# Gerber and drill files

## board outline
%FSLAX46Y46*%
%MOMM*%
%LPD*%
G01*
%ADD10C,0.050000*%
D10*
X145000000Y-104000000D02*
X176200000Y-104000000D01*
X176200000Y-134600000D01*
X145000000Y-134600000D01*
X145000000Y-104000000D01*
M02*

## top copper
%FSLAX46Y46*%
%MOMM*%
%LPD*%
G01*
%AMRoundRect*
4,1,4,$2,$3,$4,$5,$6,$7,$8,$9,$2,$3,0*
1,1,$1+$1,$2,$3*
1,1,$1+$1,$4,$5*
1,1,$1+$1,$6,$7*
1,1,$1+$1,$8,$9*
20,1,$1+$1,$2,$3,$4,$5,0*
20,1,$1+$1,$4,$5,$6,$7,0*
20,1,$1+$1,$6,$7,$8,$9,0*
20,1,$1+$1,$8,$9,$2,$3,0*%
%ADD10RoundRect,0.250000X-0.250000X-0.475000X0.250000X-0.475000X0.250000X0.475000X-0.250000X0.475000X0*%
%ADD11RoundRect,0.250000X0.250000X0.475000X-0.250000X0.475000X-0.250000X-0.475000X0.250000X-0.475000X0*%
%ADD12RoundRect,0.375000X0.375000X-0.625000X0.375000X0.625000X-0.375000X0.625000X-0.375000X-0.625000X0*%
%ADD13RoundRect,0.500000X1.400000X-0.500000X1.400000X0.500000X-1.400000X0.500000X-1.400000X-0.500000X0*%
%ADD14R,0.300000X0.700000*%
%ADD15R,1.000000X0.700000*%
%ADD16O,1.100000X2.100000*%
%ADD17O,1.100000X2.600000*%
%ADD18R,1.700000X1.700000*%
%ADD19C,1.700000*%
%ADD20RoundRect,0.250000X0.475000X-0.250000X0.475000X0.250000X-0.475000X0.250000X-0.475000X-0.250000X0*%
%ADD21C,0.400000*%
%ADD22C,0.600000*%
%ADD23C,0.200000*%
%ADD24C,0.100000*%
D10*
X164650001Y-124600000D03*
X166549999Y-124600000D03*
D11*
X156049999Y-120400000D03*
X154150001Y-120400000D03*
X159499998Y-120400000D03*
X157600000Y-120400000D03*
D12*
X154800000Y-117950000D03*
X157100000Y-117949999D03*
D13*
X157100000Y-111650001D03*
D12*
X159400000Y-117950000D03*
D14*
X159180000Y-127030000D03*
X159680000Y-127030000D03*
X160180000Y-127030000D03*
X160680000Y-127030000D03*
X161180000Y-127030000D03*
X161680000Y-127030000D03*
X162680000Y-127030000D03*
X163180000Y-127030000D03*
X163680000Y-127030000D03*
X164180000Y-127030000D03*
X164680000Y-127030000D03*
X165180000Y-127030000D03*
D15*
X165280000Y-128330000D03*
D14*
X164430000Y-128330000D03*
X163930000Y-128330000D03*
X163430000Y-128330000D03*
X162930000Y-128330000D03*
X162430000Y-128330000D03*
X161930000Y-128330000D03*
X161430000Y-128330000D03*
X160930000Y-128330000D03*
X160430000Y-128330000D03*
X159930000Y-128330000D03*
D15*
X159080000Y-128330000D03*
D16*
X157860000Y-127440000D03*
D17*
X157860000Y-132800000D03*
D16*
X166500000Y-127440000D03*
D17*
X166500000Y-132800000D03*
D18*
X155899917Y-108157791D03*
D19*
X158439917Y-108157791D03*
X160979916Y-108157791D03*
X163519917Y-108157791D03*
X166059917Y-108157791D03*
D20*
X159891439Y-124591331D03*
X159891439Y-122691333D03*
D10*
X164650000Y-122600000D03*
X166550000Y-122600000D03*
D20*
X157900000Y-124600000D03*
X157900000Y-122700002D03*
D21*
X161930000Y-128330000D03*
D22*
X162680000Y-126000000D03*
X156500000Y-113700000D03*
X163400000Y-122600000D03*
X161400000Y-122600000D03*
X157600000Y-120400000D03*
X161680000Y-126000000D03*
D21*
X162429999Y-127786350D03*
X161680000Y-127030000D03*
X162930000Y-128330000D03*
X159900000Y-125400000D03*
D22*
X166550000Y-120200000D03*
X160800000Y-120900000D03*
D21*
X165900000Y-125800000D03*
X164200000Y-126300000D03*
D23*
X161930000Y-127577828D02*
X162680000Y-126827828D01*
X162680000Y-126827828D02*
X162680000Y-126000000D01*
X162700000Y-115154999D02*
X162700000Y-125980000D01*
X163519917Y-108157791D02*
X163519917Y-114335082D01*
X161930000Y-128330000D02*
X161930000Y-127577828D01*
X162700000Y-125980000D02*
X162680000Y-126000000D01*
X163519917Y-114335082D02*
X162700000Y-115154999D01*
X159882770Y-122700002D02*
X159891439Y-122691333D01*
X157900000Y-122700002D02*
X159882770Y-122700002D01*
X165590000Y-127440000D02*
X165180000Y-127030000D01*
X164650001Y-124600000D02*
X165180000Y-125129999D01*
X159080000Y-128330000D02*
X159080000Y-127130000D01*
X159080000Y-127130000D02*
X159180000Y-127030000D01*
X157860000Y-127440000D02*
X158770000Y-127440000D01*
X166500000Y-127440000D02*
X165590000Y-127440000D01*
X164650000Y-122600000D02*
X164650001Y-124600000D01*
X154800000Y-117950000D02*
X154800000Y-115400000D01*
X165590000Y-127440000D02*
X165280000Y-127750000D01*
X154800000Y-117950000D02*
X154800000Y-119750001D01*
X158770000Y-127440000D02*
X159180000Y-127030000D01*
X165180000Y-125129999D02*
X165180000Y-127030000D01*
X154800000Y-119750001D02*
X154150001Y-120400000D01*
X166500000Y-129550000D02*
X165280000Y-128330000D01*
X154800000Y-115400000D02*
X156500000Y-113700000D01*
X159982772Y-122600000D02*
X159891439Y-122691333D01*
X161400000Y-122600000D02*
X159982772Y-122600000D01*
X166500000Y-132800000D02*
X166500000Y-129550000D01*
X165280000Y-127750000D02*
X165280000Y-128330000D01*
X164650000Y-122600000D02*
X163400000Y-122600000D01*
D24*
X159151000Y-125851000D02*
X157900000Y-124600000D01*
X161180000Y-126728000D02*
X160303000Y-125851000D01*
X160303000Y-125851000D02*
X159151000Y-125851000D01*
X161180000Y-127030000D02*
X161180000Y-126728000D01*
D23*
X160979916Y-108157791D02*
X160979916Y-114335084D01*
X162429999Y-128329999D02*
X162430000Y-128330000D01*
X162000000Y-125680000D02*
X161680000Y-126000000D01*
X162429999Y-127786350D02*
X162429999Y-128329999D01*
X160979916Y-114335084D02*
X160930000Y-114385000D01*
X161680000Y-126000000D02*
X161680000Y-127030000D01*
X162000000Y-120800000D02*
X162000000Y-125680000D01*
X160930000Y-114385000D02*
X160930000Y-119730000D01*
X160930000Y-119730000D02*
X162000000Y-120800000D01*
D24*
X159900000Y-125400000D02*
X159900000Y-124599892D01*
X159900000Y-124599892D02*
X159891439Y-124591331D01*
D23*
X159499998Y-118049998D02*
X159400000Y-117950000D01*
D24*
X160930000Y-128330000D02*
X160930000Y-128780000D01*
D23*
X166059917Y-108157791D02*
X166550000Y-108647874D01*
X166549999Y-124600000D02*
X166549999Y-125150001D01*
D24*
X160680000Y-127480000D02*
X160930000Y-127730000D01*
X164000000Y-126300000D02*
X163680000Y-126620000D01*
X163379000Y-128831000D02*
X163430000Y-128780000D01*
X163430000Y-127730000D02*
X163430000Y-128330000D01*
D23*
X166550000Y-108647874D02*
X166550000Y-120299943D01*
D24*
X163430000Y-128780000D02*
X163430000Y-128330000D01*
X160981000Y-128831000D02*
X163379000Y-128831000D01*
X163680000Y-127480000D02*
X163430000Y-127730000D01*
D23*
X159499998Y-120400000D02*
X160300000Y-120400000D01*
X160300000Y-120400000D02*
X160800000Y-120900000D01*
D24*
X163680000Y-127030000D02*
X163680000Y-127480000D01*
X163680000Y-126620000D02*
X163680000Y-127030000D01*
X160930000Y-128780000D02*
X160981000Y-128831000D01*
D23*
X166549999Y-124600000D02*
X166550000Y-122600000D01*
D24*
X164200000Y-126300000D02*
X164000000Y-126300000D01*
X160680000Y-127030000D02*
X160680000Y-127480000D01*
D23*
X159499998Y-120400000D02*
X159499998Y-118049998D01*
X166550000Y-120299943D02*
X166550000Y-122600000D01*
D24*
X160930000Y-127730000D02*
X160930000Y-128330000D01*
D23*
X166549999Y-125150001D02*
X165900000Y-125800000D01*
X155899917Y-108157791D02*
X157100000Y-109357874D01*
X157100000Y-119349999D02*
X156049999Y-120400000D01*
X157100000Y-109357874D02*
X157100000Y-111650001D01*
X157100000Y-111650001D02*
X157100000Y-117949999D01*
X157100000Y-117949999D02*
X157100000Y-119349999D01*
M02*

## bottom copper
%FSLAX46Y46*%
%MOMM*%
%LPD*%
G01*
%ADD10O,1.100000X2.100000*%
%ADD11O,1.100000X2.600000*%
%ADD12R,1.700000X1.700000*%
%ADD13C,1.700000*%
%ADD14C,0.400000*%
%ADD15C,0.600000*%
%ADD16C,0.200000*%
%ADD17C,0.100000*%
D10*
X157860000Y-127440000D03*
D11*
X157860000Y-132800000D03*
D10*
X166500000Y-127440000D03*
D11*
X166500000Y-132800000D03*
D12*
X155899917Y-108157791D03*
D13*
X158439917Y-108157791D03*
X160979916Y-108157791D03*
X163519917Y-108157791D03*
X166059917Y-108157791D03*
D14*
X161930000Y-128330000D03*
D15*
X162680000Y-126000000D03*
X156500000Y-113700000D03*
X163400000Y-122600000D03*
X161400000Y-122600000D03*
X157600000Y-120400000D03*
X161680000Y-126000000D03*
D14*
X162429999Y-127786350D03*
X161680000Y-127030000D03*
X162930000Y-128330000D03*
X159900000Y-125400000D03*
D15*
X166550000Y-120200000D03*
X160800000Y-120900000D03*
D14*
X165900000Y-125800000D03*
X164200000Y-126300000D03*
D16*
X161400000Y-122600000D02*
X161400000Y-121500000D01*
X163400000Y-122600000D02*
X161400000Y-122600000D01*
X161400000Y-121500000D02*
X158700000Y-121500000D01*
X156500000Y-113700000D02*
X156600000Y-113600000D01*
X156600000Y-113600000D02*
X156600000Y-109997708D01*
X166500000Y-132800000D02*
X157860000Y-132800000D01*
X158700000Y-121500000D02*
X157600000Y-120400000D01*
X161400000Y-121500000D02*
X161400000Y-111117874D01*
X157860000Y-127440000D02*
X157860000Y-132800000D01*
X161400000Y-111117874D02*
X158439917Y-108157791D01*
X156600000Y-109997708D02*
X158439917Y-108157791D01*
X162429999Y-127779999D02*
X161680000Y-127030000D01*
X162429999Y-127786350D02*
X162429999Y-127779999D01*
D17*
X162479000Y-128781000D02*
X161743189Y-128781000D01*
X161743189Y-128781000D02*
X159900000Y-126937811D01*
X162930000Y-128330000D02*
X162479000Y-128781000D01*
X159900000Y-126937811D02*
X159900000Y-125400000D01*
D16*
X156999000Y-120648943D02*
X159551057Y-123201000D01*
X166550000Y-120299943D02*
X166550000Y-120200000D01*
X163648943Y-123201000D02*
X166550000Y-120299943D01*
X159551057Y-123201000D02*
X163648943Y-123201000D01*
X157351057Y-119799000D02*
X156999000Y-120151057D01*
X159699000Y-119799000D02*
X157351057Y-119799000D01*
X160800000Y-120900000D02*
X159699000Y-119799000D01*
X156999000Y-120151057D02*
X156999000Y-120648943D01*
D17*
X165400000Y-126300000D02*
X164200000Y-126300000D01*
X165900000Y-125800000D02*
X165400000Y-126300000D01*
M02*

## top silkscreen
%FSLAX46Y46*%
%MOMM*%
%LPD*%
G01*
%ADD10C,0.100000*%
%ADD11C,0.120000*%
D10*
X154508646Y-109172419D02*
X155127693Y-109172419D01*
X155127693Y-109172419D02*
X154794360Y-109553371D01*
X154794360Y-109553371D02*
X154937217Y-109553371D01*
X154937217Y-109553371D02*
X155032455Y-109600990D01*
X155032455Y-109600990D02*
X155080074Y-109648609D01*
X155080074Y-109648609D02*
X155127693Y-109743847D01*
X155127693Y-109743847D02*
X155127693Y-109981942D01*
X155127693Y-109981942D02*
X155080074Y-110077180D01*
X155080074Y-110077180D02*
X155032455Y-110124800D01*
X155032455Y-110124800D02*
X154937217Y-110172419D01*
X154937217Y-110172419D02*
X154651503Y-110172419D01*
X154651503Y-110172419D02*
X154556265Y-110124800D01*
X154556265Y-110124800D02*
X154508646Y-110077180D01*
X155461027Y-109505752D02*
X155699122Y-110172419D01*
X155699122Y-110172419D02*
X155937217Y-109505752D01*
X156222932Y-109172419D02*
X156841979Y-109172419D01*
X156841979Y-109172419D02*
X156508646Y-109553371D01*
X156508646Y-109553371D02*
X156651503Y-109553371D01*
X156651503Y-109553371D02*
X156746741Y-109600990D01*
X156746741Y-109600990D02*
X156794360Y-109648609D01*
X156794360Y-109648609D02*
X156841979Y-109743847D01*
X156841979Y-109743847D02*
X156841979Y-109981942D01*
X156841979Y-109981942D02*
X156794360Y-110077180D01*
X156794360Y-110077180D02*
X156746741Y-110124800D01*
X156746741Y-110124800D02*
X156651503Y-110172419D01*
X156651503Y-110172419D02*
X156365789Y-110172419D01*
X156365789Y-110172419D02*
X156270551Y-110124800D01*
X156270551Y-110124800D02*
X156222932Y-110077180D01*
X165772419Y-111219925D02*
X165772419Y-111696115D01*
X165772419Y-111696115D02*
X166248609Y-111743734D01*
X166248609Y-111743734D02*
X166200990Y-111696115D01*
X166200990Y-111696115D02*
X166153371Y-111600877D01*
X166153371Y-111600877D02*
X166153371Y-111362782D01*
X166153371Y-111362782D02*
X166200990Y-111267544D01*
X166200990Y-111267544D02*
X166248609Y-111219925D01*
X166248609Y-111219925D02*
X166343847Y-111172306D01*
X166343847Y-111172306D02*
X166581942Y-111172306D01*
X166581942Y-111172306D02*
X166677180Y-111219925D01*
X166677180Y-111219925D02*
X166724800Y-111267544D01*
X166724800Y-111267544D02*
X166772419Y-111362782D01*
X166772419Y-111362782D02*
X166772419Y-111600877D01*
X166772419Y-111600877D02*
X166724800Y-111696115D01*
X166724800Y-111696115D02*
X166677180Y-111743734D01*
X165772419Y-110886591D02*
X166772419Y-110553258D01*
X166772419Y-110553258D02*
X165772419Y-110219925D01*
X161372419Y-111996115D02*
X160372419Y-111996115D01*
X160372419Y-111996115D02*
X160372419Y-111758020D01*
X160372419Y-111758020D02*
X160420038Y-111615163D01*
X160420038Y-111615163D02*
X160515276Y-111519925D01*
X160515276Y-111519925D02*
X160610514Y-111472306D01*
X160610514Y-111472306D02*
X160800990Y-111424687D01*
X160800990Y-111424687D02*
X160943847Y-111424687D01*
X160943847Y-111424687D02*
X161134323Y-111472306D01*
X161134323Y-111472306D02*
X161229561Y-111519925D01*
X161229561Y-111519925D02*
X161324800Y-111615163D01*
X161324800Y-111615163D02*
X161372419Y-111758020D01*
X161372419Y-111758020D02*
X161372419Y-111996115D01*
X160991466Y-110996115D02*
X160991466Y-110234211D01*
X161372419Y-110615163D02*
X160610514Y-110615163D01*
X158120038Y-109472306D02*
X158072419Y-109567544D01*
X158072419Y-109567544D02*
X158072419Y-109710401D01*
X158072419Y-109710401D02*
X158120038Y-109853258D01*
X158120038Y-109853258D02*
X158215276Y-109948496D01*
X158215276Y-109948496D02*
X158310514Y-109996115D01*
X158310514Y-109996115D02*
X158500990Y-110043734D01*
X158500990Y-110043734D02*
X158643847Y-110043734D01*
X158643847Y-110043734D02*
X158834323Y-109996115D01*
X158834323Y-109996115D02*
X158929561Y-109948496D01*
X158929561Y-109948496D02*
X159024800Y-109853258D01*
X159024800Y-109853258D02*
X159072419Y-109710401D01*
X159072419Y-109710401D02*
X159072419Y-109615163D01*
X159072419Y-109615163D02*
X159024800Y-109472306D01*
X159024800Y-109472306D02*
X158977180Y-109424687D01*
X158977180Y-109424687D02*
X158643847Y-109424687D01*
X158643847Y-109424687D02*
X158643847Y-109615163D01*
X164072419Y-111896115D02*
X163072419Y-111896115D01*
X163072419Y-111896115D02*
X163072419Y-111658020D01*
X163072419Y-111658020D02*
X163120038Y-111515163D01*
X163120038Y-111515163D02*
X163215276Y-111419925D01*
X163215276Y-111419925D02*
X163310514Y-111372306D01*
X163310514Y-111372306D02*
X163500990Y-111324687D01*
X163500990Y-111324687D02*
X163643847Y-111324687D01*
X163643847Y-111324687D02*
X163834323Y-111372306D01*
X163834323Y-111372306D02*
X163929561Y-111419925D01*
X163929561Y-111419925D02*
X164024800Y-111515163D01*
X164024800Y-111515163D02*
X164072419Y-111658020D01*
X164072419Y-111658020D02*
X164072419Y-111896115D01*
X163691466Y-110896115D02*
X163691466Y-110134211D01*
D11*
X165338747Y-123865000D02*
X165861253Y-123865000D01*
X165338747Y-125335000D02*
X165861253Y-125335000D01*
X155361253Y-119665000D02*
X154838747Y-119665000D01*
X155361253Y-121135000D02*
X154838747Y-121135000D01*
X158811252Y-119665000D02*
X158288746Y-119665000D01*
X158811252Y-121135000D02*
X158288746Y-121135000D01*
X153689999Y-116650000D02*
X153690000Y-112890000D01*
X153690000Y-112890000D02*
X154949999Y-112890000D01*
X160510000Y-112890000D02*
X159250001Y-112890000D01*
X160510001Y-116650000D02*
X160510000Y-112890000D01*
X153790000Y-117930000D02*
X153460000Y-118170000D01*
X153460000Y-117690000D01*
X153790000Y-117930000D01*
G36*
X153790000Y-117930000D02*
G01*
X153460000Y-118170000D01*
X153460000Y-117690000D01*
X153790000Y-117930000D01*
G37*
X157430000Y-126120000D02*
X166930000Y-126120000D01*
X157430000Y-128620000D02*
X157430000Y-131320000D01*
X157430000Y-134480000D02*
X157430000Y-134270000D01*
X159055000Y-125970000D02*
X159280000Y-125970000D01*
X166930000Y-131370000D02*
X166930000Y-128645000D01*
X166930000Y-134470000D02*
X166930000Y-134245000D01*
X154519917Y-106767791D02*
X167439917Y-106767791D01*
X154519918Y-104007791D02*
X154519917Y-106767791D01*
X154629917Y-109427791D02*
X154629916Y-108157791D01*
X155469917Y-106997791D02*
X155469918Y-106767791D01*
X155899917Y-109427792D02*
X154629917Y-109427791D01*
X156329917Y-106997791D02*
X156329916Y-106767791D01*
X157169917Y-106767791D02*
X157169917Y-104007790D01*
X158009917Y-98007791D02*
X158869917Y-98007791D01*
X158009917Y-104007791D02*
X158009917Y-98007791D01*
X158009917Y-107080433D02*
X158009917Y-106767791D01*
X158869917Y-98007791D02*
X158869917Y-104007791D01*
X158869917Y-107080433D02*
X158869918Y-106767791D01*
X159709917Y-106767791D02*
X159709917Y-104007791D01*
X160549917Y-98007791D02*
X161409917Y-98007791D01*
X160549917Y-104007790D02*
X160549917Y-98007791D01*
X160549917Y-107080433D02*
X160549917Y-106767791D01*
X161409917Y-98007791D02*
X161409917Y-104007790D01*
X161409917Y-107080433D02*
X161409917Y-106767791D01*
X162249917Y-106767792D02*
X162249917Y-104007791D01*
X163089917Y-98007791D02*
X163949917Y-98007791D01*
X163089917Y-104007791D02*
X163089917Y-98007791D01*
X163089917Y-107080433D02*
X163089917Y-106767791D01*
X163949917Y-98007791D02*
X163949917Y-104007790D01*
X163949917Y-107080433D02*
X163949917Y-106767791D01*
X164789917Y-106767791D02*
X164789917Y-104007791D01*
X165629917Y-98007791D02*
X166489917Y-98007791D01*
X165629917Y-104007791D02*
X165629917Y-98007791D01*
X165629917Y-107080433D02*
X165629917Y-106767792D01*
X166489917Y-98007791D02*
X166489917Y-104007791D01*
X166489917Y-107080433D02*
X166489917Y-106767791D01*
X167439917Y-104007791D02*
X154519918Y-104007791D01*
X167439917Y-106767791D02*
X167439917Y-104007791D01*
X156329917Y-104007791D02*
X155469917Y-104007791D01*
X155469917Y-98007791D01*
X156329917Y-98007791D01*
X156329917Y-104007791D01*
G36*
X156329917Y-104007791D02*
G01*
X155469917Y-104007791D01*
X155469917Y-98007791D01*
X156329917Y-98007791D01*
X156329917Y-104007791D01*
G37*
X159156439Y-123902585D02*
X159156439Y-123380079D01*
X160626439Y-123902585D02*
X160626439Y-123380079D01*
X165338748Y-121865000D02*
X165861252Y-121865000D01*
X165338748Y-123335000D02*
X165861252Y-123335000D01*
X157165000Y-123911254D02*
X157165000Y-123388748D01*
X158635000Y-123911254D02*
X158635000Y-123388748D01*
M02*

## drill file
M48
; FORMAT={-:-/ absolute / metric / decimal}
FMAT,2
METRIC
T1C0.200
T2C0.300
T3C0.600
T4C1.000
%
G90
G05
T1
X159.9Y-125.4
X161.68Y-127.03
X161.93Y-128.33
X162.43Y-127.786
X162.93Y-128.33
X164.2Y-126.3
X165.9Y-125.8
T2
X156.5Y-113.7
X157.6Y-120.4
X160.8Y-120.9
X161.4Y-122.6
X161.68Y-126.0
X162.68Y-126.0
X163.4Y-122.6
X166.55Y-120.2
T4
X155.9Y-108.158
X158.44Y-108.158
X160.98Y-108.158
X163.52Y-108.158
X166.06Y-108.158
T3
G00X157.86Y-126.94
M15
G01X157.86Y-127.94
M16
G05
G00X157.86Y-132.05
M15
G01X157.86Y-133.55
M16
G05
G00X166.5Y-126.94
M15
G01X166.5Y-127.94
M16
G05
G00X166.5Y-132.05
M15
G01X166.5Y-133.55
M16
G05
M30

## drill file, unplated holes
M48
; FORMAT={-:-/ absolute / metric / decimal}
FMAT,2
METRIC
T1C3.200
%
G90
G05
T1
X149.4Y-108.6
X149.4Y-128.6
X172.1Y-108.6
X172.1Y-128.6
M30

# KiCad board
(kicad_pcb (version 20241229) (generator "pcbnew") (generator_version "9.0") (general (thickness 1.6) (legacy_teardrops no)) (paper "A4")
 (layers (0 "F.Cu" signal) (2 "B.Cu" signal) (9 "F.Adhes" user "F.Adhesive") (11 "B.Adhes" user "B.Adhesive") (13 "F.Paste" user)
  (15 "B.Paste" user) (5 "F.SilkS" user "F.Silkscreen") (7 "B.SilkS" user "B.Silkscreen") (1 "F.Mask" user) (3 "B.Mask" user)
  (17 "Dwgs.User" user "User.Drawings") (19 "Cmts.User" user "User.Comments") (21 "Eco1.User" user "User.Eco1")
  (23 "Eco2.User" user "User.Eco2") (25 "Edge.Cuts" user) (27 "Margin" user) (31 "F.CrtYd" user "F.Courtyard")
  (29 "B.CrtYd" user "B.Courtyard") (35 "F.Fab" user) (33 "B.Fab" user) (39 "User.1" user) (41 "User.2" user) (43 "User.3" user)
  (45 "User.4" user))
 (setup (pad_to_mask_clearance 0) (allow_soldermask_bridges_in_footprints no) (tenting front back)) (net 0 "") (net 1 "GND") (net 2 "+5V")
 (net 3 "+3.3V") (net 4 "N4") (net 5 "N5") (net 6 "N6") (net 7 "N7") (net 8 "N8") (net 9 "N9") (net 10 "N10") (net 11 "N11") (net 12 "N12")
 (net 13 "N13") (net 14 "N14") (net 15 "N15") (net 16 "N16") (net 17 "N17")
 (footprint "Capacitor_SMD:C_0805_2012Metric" (layer "F.Cu") (at 165.6 124.6)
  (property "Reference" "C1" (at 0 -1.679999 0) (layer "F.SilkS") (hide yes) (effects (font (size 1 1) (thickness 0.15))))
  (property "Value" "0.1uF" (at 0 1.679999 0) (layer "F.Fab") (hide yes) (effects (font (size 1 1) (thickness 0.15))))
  (fp_line (start -0.261253 -0.735) (end 0.261253 -0.735) (stroke (width 0.12) (type solid)) (layer "F.SilkS"))
  (fp_line (start -0.261253 0.735) (end 0.261253 0.735) (stroke (width 0.12) (type solid)) (layer "F.SilkS"))
  (pad "1" smd roundrect (at -0.949999 0) (size 1 1.45) (layers "F.Cu" "F.Mask" "F.Paste") (roundrect_rratio 0.25) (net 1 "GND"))
  (pad "2" smd roundrect (at 0.949999 0) (size 1 1.45) (layers "F.Cu" "F.Mask" "F.Paste") (roundrect_rratio 0.25) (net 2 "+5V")))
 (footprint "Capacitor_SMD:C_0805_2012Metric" (layer "F.Cu") (at 155.1 120.4 180)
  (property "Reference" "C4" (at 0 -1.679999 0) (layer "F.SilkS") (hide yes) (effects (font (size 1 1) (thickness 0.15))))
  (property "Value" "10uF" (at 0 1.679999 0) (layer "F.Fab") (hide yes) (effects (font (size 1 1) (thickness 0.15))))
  (fp_line (start -0.261253 0.735) (end 0.261253 0.735) (stroke (width 0.12) (type solid)) (layer "F.SilkS"))
  (fp_line (start -0.261253 -0.735) (end 0.261253 -0.735) (stroke (width 0.12) (type solid)) (layer "F.SilkS"))
  (pad "1" smd roundrect (at -0.949999 0 180) (size 1 1.45) (layers "F.Cu" "F.Mask" "F.Paste") (roundrect_rratio 0.25) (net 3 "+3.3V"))
  (pad "2" smd roundrect (at 0.949999 0 180) (size 1 1.45) (layers "F.Cu" "F.Mask" "F.Paste") (roundrect_rratio 0.25) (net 1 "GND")))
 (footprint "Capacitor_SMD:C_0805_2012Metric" (layer "F.Cu") (at 158.549999 120.4 180)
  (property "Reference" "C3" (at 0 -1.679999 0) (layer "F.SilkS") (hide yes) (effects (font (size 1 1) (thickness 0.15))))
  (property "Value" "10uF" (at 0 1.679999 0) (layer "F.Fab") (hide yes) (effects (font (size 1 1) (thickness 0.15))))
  (fp_line (start -0.261253 0.735) (end 0.261253 0.735) (stroke (width 0.12) (type solid)) (layer "F.SilkS"))
  (fp_line (start -0.261253 -0.735) (end 0.261253 -0.735) (stroke (width 0.12) (type solid)) (layer "F.SilkS"))
  (pad "1" smd roundrect (at -0.949999 0 180) (size 1 1.45) (layers "F.Cu" "F.Mask" "F.Paste") (roundrect_rratio 0.25) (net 2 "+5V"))
  (pad "2" smd roundrect (at 0.949999 0 180) (size 1 1.45) (layers "F.Cu" "F.Mask" "F.Paste") (roundrect_rratio 0.25) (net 1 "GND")))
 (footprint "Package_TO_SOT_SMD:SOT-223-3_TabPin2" (layer "F.Cu") (at 157.1 114.8 90)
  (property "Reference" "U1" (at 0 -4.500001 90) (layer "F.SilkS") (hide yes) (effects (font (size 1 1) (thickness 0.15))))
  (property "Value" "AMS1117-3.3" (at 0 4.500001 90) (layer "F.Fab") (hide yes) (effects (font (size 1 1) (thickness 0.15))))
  (fp_line (start -1.85 -3.410001) (end 1.91 -3.41) (stroke (width 0.12) (type solid)) (layer "F.SilkS"))
  (fp_line (start 1.91 -3.41) (end 1.91 -2.150001) (stroke (width 0.12) (type solid)) (layer "F.SilkS"))
  (fp_line (start 1.91 3.41) (end 1.91 2.150001) (stroke (width 0.12) (type solid)) (layer "F.SilkS"))
  (fp_line (start -1.85 3.410001) (end 1.91 3.41) (stroke (width 0.12) (type solid)) (layer "F.SilkS"))
  (fp_poly
   (pts (xy -3.13 -3.31) (xy -3.37 -3.64) (xy -2.89 -3.64) (xy -3.13 -3.31)) (stroke (width 0.12) (type solid)) (fill yes) (layer "F.SilkS"))
  (pad "1" smd roundrect (at -3.15 -2.3 90) (size 2 1.5) (layers "F.Cu" "F.Mask" "F.Paste") (roundrect_rratio 0.25) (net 1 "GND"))
  (pad "2" smd roundrect (at -3.149999 0 90) (size 2 1.5) (layers "F.Cu" "F.Mask" "F.Paste") (roundrect_rratio 0.25) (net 3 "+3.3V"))
  (pad "2" smd roundrect (at 3.149999 0 90) (size 2 3.8) (layers "F.Cu" "F.Mask" "F.Paste") (roundrect_rratio 0.25) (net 3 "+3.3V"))
  (pad "3" smd roundrect (at -3.15 2.3 90) (size 2 1.5) (layers "F.Cu" "F.Mask" "F.Paste") (roundrect_rratio 0.25) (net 2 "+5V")))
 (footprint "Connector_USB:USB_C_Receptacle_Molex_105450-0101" (layer "F.Cu") (at 162.18 130.245)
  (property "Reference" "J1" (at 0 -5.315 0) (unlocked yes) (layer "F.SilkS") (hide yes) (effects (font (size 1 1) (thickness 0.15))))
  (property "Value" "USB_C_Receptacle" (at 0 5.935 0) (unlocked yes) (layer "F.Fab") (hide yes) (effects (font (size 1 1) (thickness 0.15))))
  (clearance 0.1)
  (fp_line (start -4.75 -4.125) (end 4.75 -4.125) (stroke (width 0.12) (type solid)) (layer "F.SilkS"))
  (fp_line (start -4.75 -1.625) (end -4.75 1.075) (stroke (width 0.12) (type solid)) (layer "F.SilkS"))
  (fp_line (start -4.75 4.235) (end -4.75 4.025) (stroke (width 0.12) (type solid)) (layer "F.SilkS"))
  (fp_line (start -3.125 -4.275) (end -2.9 -4.275) (stroke (width 0.12) (type solid)) (layer "F.SilkS"))
  (fp_line (start 4.75 1.125) (end 4.75 -1.6) (stroke (width 0.12) (type solid)) (layer "F.SilkS"))
  (fp_line (start 4.75 4.225) (end 4.75 4) (stroke (width 0.12) (type solid)) (layer "F.SilkS"))
  (pad "A1" smd rect (at -3 -3.215) (size 0.3 0.7) (layers "F.Cu" "F.Mask" "F.Paste") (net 1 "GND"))
  (pad "A2" smd rect (at -2.5 -3.215) (size 0.3 0.7) (layers "F.Cu" "F.Mask" "F.Paste") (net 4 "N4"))
  (pad "A3" smd rect (at -2 -3.215) (size 0.3 0.7) (layers "F.Cu" "F.Mask" "F.Paste") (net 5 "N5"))
  (pad "A4" smd rect (at -1.5 -3.215) (size 0.3 0.7) (layers "F.Cu" "F.Mask" "F.Paste") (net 2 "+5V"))
  (pad "A5" smd rect (at -1 -3.215) (size 0.3 0.7) (layers "F.Cu" "F.Mask" "F.Paste") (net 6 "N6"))
  (pad "A6" smd rect (at -0.5 -3.215) (size 0.3 0.7) (layers "F.Cu" "F.Mask" "F.Paste") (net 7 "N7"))
  (pad "A7" smd rect (at 0.5 -3.215) (size 0.3 0.7) (layers "F.Cu" "F.Mask" "F.Paste") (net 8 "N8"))
  (pad "A8" smd rect (at 1 -3.215) (size 0.3 0.7) (layers "F.Cu" "F.Mask" "F.Paste") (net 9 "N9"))
  (pad "A9" smd rect (at 1.5 -3.215) (size 0.3 0.7) (layers "F.Cu" "F.Mask" "F.Paste") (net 2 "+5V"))
  (pad "A10" smd rect (at 2 -3.215) (size 0.3 0.7) (layers "F.Cu" "F.Mask" "F.Paste") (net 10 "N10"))
  (pad "A11" smd rect (at 2.5 -3.215) (size 0.3 0.7) (layers "F.Cu" "F.Mask" "F.Paste") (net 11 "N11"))
  (pad "A12" smd rect (at 3 -3.215) (size 0.3 0.7) (layers "F.Cu" "F.Mask" "F.Paste") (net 1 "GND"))
  (pad "B1" smd rect (at 3.1 -1.915) (size 1 0.7) (layers "F.Cu" "F.Mask" "F.Paste") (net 1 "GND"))
  (pad "B2" smd rect (at 2.25 -1.915) (size 0.3 0.7) (layers "F.Cu" "F.Mask" "F.Paste") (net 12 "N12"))
  (pad "B3" smd rect (at 1.75 -1.915) (size 0.3 0.7) (layers "F.Cu" "F.Mask" "F.Paste") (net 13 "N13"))
  (pad "B4" smd rect (at 1.25 -1.915) (size 0.3 0.7) (layers "F.Cu" "F.Mask" "F.Paste") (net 2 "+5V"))
  (pad "B5" smd rect (at 0.75 -1.915) (size 0.3 0.7) (layers "F.Cu" "F.Mask" "F.Paste") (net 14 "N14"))
  (pad "B6" smd rect (at 0.25 -1.915) (size 0.3 0.7) (layers "F.Cu" "F.Mask" "F.Paste") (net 7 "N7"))
  (pad "B7" smd rect (at -0.25 -1.915) (size 0.3 0.7) (layers "F.Cu" "F.Mask" "F.Paste") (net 8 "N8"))
  (pad "B8" smd rect (at -0.75 -1.915) (size 0.3 0.7) (layers "F.Cu" "F.Mask" "F.Paste") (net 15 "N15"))
  (pad "B9" smd rect (at -1.25 -1.915) (size 0.3 0.7) (layers "F.Cu" "F.Mask" "F.Paste") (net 2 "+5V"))
  (pad "B10" smd rect (at -1.75 -1.915) (size 0.3 0.7) (layers "F.Cu" "F.Mask" "F.Paste") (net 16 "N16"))
  (pad "B11" smd rect (at -2.25 -1.915) (size 0.3 0.7) (layers "F.Cu" "F.Mask" "F.Paste") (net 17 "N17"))
  (pad "B12" smd rect (at -3.1 -1.915) (size 1 0.7) (layers "F.Cu" "F.Mask" "F.Paste") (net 1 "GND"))
  (pad "S1" thru_hole oval (at -4.32 -2.805) (size 1.1 2.1) (drill oval 0.6 1.6) (layers "*.Cu" "*.Mask") (remove_unused_layers no)
   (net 1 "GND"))
  (pad "S1" thru_hole oval (at -4.32 2.555) (size 1.1 2.6) (drill oval 0.6 2.1) (layers "*.Cu" "*.Mask") (remove_unused_layers no)
   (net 1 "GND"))
  (pad "S1" thru_hole oval (at 4.32 -2.805) (size 1.1 2.1) (drill oval 0.6 1.6) (layers "*.Cu" "*.Mask") (remove_unused_layers no)
   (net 1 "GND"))
  (pad "S1" thru_hole oval (at 4.32 2.555) (size 1.1 2.6) (drill oval 0.6 2.1) (layers "*.Cu" "*.Mask") (remove_unused_layers no)
   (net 1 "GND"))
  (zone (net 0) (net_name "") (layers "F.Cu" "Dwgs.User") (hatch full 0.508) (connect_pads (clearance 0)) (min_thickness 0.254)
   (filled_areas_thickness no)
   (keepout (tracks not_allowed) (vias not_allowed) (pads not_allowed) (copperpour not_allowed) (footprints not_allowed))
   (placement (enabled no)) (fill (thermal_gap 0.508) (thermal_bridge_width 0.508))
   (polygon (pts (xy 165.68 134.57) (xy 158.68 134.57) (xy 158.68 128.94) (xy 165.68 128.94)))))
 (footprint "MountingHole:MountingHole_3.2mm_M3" (layer "F.Cu") (at 172.1 108.6)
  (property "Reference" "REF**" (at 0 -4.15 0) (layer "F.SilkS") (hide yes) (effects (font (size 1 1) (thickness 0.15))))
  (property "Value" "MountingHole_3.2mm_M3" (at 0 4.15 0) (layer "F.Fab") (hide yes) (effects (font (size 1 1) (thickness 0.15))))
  (pad "" np_thru_hole circle (at 0 0) (size 3.2 3.2) (drill 3.2) (layers "*.Cu" "*.Mask")))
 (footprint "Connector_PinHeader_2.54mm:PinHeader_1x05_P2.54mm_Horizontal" (layer "F.Cu") (at 155.899917 108.157791 90)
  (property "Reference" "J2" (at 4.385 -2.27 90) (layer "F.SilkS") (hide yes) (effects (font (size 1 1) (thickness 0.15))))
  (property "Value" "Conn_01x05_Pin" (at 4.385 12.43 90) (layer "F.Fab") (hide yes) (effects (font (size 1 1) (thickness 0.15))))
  (fp_line (start 1.39 -1.38) (end 1.39 11.54) (stroke (width 0.12) (type solid)) (layer "F.SilkS"))
  (fp_line (start 4.15 -1.379999) (end 1.39 -1.38) (stroke (width 0.12) (type solid)) (layer "F.SilkS"))
  (fp_line (start -1.27 -1.27) (end 0 -1.270001) (stroke (width 0.12) (type solid)) (layer "F.SilkS"))
  (fp_line (start 1.16 -0.43) (end 1.39 -0.429999) (stroke (width 0.12) (type solid)) (layer "F.SilkS"))
  (fp_line (start -1.270001 0) (end -1.27 -1.27) (stroke (width 0.12) (type solid)) (layer "F.SilkS"))
  (fp_line (start 1.16 0.43) (end 1.39 0.429999) (stroke (width 0.12) (type solid)) (layer "F.SilkS"))
  (fp_line (start 1.39 1.27) (end 4.150001 1.27) (stroke (width 0.12) (type solid)) (layer "F.SilkS"))
  (fp_line (start 10.15 2.11) (end 10.15 2.97) (stroke (width 0.12) (type solid)) (layer "F.SilkS"))
  (fp_line (start 4.15 2.11) (end 10.15 2.11) (stroke (width 0.12) (type solid)) (layer "F.SilkS"))
  (fp_line (start 1.077358 2.11) (end 1.39 2.11) (stroke (width 0.12) (type solid)) (layer "F.SilkS"))
  (fp_line (start 10.15 2.97) (end 4.15 2.97) (stroke (width 0.12) (type solid)) (layer "F.SilkS"))
  (fp_line (start 1.077358 2.97) (end 1.39 2.970001) (stroke (width 0.12) (type solid)) (layer "F.SilkS"))
  (fp_line (start 1.39 3.81) (end 4.15 3.81) (stroke (width 0.12) (type solid)) (layer "F.SilkS"))
  (fp_line (start 10.15 4.65) (end 10.15 5.51) (stroke (width 0.12) (type solid)) (layer "F.SilkS"))
  (fp_line (start 4.150001 4.65) (end 10.15 4.65) (stroke (width 0.12) (type solid)) (layer "F.SilkS"))
  (fp_line (start 1.077358 4.65) (end 1.39 4.65) (stroke (width 0.12) (type solid)) (layer "F.SilkS"))
  (fp_line (start 10.15 5.51) (end 4.150001 5.51) (stroke (width 0.12) (type solid)) (layer "F.SilkS"))
  (fp_line (start 1.077358 5.51) (end 1.39 5.51) (stroke (width 0.12) (type solid)) (layer "F.SilkS"))
  (fp_line (start 1.389999 6.35) (end 4.15 6.35) (stroke (width 0.12) (type solid)) (layer "F.SilkS"))
  (fp_line (start 10.15 7.19) (end 10.15 8.05) (stroke (width 0.12) (type solid)) (layer "F.SilkS"))
  (fp_line (start 4.15 7.19) (end 10.15 7.19) (stroke (width 0.12) (type solid)) (layer "F.SilkS"))
  (fp_line (start 1.077358 7.19) (end 1.39 7.19) (stroke (width 0.12) (type solid)) (layer "F.SilkS"))
  (fp_line (start 10.15 8.05) (end 4.150001 8.05) (stroke (width 0.12) (type solid)) (layer "F.SilkS"))
  (fp_line (start 1.077358 8.05) (end 1.39 8.05) (stroke (width 0.12) (type solid)) (layer "F.SilkS"))
  (fp_line (start 1.39 8.89) (end 4.15 8.89) (stroke (width 0.12) (type solid)) (layer "F.SilkS"))
  (fp_line (start 10.15 9.73) (end 10.15 10.59) (stroke (width 0.12) (type solid)) (layer "F.SilkS"))
  (fp_line (start 4.15 9.73) (end 10.15 9.73) (stroke (width 0.12) (type solid)) (layer "F.SilkS"))
  (fp_line (start 1.077358 9.73) (end 1.389999 9.73) (stroke (width 0.12) (type solid)) (layer "F.SilkS"))
  (fp_line (start 10.15 10.59) (end 4.15 10.59) (stroke (width 0.12) (type solid)) (layer "F.SilkS"))
  (fp_line (start 1.077358 10.59) (end 1.39 10.59) (stroke (width 0.12) (type solid)) (layer "F.SilkS"))
  (fp_line (start 4.15 11.54) (end 4.15 -1.379999) (stroke (width 0.12) (type solid)) (layer "F.SilkS"))
  (fp_line (start 1.39 11.54) (end 4.15 11.54) (stroke (width 0.12) (type solid)) (layer "F.SilkS"))
  (fp_poly
   (pts (xy 4.15 -0.43) (xy 10.15 -0.43) (xy 10.15 0.43) (xy 4.15 0.43)) (stroke (width 0.12) (type solid)) (fill yes) (layer "F.SilkS"))
  (pad "1" thru_hole rect (at 0 0 90) (size 1.7 1.7) (drill 1) (layers "*.Cu" "*.Mask") (remove_unused_layers no) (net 3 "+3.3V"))
  (pad "2" thru_hole circle (at 0 2.54 90) (size 1.7 1.7) (drill 1) (layers "*.Cu" "*.Mask") (remove_unused_layers no) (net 1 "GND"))
  (pad "3" thru_hole circle (at 0 5.079999 90) (size 1.7 1.7) (drill 1) (layers "*.Cu" "*.Mask") (remove_unused_layers no) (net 7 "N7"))
  (pad "4" thru_hole circle (at 0 7.62 90) (size 1.7 1.7) (drill 1) (layers "*.Cu" "*.Mask") (remove_unused_layers no) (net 8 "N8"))
  (pad "5" thru_hole circle (at 0 10.16 90) (size 1.7 1.7) (drill 1) (layers "*.Cu" "*.Mask") (remove_unused_layers no) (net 2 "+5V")))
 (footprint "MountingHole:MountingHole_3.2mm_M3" (layer "F.Cu") (at 172.1 128.6)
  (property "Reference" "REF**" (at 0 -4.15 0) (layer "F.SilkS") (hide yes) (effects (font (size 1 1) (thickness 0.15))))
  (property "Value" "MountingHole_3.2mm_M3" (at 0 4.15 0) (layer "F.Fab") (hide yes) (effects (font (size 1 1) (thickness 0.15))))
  (pad "" np_thru_hole circle (at 0 0) (size 3.2 3.2) (drill 3.2) (layers "*.Cu" "*.Mask")))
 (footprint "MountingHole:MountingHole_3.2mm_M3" (layer "F.Cu") (at 149.4 108.6)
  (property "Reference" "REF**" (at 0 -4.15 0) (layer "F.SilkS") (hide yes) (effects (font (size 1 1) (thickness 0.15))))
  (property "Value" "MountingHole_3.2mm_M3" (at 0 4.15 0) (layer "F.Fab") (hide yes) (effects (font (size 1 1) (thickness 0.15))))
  (pad "" np_thru_hole circle (at 0 0) (size 3.2 3.2) (drill 3.2) (layers "*.Cu" "*.Mask")))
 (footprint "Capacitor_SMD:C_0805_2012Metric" (layer "F.Cu") (at 159.891439 123.641332 90)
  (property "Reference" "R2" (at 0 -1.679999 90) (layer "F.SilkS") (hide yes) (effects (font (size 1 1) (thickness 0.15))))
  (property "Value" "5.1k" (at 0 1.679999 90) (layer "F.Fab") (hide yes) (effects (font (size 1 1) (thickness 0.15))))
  (fp_line (start -0.261253 -0.735) (end 0.261253 -0.735) (stroke (width 0.12) (type solid)) (layer "F.SilkS"))
  (fp_line (start -0.261253 0.735) (end 0.261253 0.735) (stroke (width 0.12) (type solid)) (layer "F.SilkS"))
  (pad "1" smd roundrect (at -0.949999 0 90) (size 1 1.45) (layers "F.Cu" "F.Mask" "F.Paste") (roundrect_rratio 0.25) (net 14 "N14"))
  (pad "2" smd roundrect (at 0.949999 0 90) (size 1 1.45) (layers "F.Cu" "F.Mask" "F.Paste") (roundrect_rratio 0.25) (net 1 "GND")))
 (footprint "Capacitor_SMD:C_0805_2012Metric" (layer "F.Cu") (at 165.6 122.6)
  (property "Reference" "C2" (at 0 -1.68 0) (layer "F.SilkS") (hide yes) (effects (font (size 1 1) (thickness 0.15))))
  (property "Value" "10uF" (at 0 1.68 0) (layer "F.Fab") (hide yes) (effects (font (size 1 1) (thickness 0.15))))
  (fp_line (start -0.261252 -0.735) (end 0.261252 -0.735) (stroke (width 0.12) (type solid)) (layer "F.SilkS"))
  (fp_line (start -0.261252 0.735) (end 0.261252 0.735) (stroke (width 0.12) (type solid)) (layer "F.SilkS"))
  (pad "1" smd roundrect (at -0.95 0) (size 1 1.45) (layers "F.Cu" "F.Mask" "F.Paste") (roundrect_rratio 0.25) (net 1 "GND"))
  (pad "2" smd roundrect (at 0.95 0) (size 1 1.45) (layers "F.Cu" "F.Mask" "F.Paste") (roundrect_rratio 0.25) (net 2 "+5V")))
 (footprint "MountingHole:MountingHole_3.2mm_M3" (layer "F.Cu") (at 149.4 128.6)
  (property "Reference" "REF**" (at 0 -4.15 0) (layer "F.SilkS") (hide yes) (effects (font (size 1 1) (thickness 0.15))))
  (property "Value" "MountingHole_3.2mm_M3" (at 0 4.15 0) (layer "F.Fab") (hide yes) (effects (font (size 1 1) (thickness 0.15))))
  (pad "" np_thru_hole circle (at 0 0) (size 3.2 3.2) (drill 3.2) (layers "*.Cu" "*.Mask")))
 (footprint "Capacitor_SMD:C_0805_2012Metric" (layer "F.Cu") (at 157.9 123.650001 90)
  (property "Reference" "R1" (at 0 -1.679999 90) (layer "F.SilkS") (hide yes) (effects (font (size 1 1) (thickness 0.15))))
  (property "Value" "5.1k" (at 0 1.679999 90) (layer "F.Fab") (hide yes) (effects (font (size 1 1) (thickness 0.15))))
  (fp_line (start -0.261253 -0.735) (end 0.261253 -0.735) (stroke (width 0.12) (type solid)) (layer "F.SilkS"))
  (fp_line (start -0.261253 0.735) (end 0.261253 0.735) (stroke (width 0.12) (type solid)) (layer "F.SilkS"))
  (pad "1" smd roundrect (at -0.949999 0 90) (size 1 1.45) (layers "F.Cu" "F.Mask" "F.Paste") (roundrect_rratio 0.25) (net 6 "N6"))
  (pad "2" smd roundrect (at 0.949999 0 90) (size 1 1.45) (layers "F.Cu" "F.Mask" "F.Paste") (roundrect_rratio 0.25) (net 1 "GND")))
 (gr_rect (start 145 104) (end 176.2 134.6) (stroke (width 0.05) (type default)) (fill no) (layer "Edge.Cuts"))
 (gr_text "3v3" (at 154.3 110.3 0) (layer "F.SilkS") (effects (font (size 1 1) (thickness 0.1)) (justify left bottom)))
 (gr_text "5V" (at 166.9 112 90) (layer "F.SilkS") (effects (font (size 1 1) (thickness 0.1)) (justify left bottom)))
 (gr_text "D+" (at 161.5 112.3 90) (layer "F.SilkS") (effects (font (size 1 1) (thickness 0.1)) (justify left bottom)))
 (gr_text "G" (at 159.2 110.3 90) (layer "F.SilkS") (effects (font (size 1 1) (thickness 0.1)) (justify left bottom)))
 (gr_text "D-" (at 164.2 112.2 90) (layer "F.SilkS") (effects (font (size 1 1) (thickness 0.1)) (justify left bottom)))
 (segment (start 161.93 127.577828) (end 162.68 126.827828) (width 0.2) (layer "F.Cu") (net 8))
 (segment (start 162.68 126.827828) (end 162.68 126) (width 0.2) (layer "F.Cu") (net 8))
 (segment (start 162.7 115.154999) (end 162.7 125.98) (width 0.2) (layer "F.Cu") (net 8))
 (segment (start 163.519917 108.157791) (end 163.519917 114.335082) (width 0.2) (layer "F.Cu") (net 8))
 (segment (start 161.93 128.33) (end 161.93 127.577828) (width 0.2) (layer "F.Cu") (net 8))
 (segment (start 162.7 125.98) (end 162.68 126) (width 0.2) (layer "F.Cu") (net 8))
 (segment (start 163.519917 114.335082) (end 162.7 115.154999) (width 0.2) (layer "F.Cu") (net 8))
 (via (at 161.93 128.33) (size 0.4) (drill 0.2) (layers "F.Cu" "B.Cu") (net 8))
 (via (at 162.68 126) (size 0.6) (drill 0.3) (layers "F.Cu" "B.Cu") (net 8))
 (segment (start 159.88277 122.700002) (end 159.891439 122.691333) (width 0.2) (layer "F.Cu") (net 1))
 (segment (start 157.9 122.700002) (end 159.88277 122.700002) (width 0.2) (layer "F.Cu") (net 1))
 (segment (start 165.59 127.44) (end 165.18 127.03) (width 0.2) (layer "F.Cu") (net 1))
 (segment (start 164.650001 124.6) (end 165.18 125.129999) (width 0.2) (layer "F.Cu") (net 1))
 (segment (start 159.08 128.33) (end 159.08 127.13) (width 0.2) (layer "F.Cu") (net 1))
 (segment (start 159.08 127.13) (end 159.18 127.03) (width 0.2) (layer "F.Cu") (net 1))
 (segment (start 157.86 127.44) (end 158.77 127.44) (width 0.2) (layer "F.Cu") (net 1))
 (segment (start 166.5 127.44) (end 165.59 127.44) (width 0.2) (layer "F.Cu") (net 1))
 (segment (start 164.65 122.6) (end 164.650001 124.6) (width 0.2) (layer "F.Cu") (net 1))
 (segment (start 154.8 117.95) (end 154.8 115.4) (width 0.2) (layer "F.Cu") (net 1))
 (segment (start 165.59 127.44) (end 165.28 127.75) (width 0.2) (layer "F.Cu") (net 1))
 (segment (start 154.8 117.95) (end 154.8 119.750001) (width 0.2) (layer "F.Cu") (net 1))
 (segment (start 158.77 127.44) (end 159.18 127.03) (width 0.2) (layer "F.Cu") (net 1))
 (segment (start 165.18 125.129999) (end 165.18 127.03) (width 0.2) (layer "F.Cu") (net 1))
 (segment (start 154.8 119.750001) (end 154.150001 120.4) (width 0.2) (layer "F.Cu") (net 1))
 (segment (start 166.5 129.55) (end 165.28 128.33) (width 0.2) (layer "F.Cu") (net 1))
 (segment (start 154.8 115.4) (end 156.5 113.7) (width 0.2) (layer "F.Cu") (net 1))
 (segment (start 159.982772 122.6) (end 159.891439 122.691333) (width 0.2) (layer "F.Cu") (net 1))
 (segment (start 161.4 122.6) (end 159.982772 122.6) (width 0.2) (layer "F.Cu") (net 1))
 (segment (start 166.5 132.8) (end 166.5 129.55) (width 0.2) (layer "F.Cu") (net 1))
 (segment (start 165.28 127.75) (end 165.28 128.33) (width 0.2) (layer "F.Cu") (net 1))
 (segment (start 164.65 122.6) (end 163.4 122.6) (width 0.2) (layer "F.Cu") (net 1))
 (via (at 156.5 113.7) (size 0.6) (drill 0.3) (layers "F.Cu" "B.Cu") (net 1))
 (via (at 163.4 122.6) (size 0.6) (drill 0.3) (layers "F.Cu" "B.Cu") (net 1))
 (via (at 161.4 122.6) (size 0.6) (drill 0.3) (layers "F.Cu" "B.Cu") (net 1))
 (via (at 157.6 120.4) (size 0.6) (drill 0.3) (layers "F.Cu" "B.Cu") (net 1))
 (segment (start 161.4 122.6) (end 161.4 121.5) (width 0.2) (layer "B.Cu") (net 1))
 (segment (start 163.4 122.6) (end 161.4 122.6) (width 0.2) (layer "B.Cu") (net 1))
 (segment (start 161.4 121.5) (end 158.7 121.5) (width 0.2) (layer "B.Cu") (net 1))
 (segment (start 156.5 113.7) (end 156.6 113.6) (width 0.2) (layer "B.Cu") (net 1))
 (segment (start 156.6 113.6) (end 156.6 109.997708) (width 0.2) (layer "B.Cu") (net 1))
 (segment (start 166.5 132.8) (end 157.86 132.8) (width 0.2) (layer "B.Cu") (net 1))
 (segment (start 158.7 121.5) (end 157.6 120.4) (width 0.2) (layer "B.Cu") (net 1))
 (segment (start 161.4 121.5) (end 161.4 111.117874) (width 0.2) (layer "B.Cu") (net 1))
 (segment (start 157.86 127.44) (end 157.86 132.8) (width 0.2) (layer "B.Cu") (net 1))
 (segment (start 161.4 111.117874) (end 158.439917 108.157791) (width 0.2) (layer "B.Cu") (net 1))
 (segment (start 156.6 109.997708) (end 158.439917 108.157791) (width 0.2) (layer "B.Cu") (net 1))
 (segment (start 159.151 125.851) (end 157.9 124.6) (width 0.1) (layer "F.Cu") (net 6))
 (segment (start 161.18 126.728) (end 160.303 125.851) (width 0.1) (layer "F.Cu") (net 6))
 (segment (start 160.303 125.851) (end 159.151 125.851) (width 0.1) (layer "F.Cu") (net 6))
 (segment (start 161.18 127.03) (end 161.18 126.728) (width 0.1) (layer "F.Cu") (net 6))
 (segment (start 160.979916 108.157791) (end 160.979916 114.335084) (width 0.2) (layer "F.Cu") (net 7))
 (segment (start 162.429999 128.329999) (end 162.43 128.33) (width 0.2) (layer "F.Cu") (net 7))
 (segment (start 162 125.68) (end 161.68 126) (width 0.2) (layer "F.Cu") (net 7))
 (segment (start 162.429999 127.78635) (end 162.429999 128.329999) (width 0.2) (layer "F.Cu") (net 7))
 (segment (start 160.979916 114.335084) (end 160.93 114.385) (width 0.2) (layer "F.Cu") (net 7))
 (segment (start 161.68 126) (end 161.68 127.03) (width 0.2) (layer "F.Cu") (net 7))
 (segment (start 162 120.8) (end 162 125.68) (width 0.2) (layer "F.Cu") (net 7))
 (segment (start 160.93 114.385) (end 160.93 119.73) (width 0.2) (layer "F.Cu") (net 7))
 (segment (start 160.93 119.73) (end 162 120.8) (width 0.2) (layer "F.Cu") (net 7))
 (via (at 161.68 126) (size 0.6) (drill 0.3) (layers "F.Cu" "B.Cu") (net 7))
 (via (at 162.429999 127.78635) (size 0.4) (drill 0.2) (layers "F.Cu" "B.Cu") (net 7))
 (via (at 161.68 127.03) (size 0.4) (drill 0.2) (layers "F.Cu" "B.Cu") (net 7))
 (segment (start 162.429999 127.779999) (end 161.68 127.03) (width 0.2) (layer "B.Cu") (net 7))
 (segment (start 162.429999 127.78635) (end 162.429999 127.779999) (width 0.2) (layer "B.Cu") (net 7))
 (segment (start 159.9 125.4) (end 159.9 124.599892) (width 0.1) (layer "F.Cu") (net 14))
 (segment (start 159.9 124.599892) (end 159.891439 124.591331) (width 0.1) (layer "F.Cu") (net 14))
 (via (at 162.93 128.33) (size 0.4) (drill 0.2) (layers "F.Cu" "B.Cu") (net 14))
 (via (at 159.9 125.4) (size 0.4) (drill 0.2) (layers "F.Cu" "B.Cu") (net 14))
 (segment (start 162.479 128.781) (end 161.743189 128.781) (width 0.1) (layer "B.Cu") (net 14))
 (segment (start 161.743189 128.781) (end 159.9 126.937811) (width 0.1) (layer "B.Cu") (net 14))
 (segment (start 162.93 128.33) (end 162.479 128.781) (width 0.1) (layer "B.Cu") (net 14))
 (segment (start 159.9 126.937811) (end 159.9 125.4) (width 0.1) (layer "B.Cu") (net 14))
 (segment (start 159.499998 118.049998) (end 159.4 117.95) (width 0.2) (layer "F.Cu") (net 2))
 (segment (start 160.93 128.33) (end 160.93 128.78) (width 0.1) (layer "F.Cu") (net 2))
 (segment (start 166.059917 108.157791) (end 166.55 108.647874) (width 0.2) (layer "F.Cu") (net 2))
 (segment (start 166.549999 124.6) (end 166.549999 125.150001) (width 0.2) (layer "F.Cu") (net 2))
 (segment (start 160.68 127.48) (end 160.93 127.73) (width 0.1) (layer "F.Cu") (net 2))
 (segment (start 164 126.3) (end 163.68 126.62) (width 0.1) (layer "F.Cu") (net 2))
 (segment (start 163.379 128.831) (end 163.43 128.78) (width 0.1) (layer "F.Cu") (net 2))
 (segment (start 163.43 127.73) (end 163.43 128.33) (width 0.1) (layer "F.Cu") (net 2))
 (segment (start 166.55 108.647874) (end 166.55 120.299943) (width 0.2) (layer "F.Cu") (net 2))
 (segment (start 163.43 128.78) (end 163.43 128.33) (width 0.1) (layer "F.Cu") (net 2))
 (segment (start 160.981 128.831) (end 163.379 128.831) (width 0.1) (layer "F.Cu") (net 2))
 (segment (start 163.68 127.48) (end 163.43 127.73) (width 0.1) (layer "F.Cu") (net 2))
 (segment (start 159.499998 120.4) (end 160.3 120.4) (width 0.2) (layer "F.Cu") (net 2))
 (segment (start 160.3 120.4) (end 160.8 120.9) (width 0.2) (layer "F.Cu") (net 2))
 (segment (start 163.68 127.03) (end 163.68 127.48) (width 0.1) (layer "F.Cu") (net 2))
 (segment (start 163.68 126.62) (end 163.68 127.03) (width 0.1) (layer "F.Cu") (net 2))
 (segment (start 160.93 128.78) (end 160.981 128.831) (width 0.1) (layer "F.Cu") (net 2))
 (segment (start 166.549999 124.6) (end 166.55 122.6) (width 0.2) (layer "F.Cu") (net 2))
 (segment (start 164.2 126.3) (end 164 126.3) (width 0.1) (layer "F.Cu") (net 2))
 (segment (start 160.68 127.03) (end 160.68 127.48) (width 0.1) (layer "F.Cu") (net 2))
 (segment (start 159.499998 120.4) (end 159.499998 118.049998) (width 0.2) (layer "F.Cu") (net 2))
 (segment (start 166.55 120.299943) (end 166.55 122.6) (width 0.2) (layer "F.Cu") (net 2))
 (segment (start 160.93 127.73) (end 160.93 128.33) (width 0.1) (layer "F.Cu") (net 2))
 (segment (start 166.549999 125.150001) (end 165.9 125.8) (width 0.2) (layer "F.Cu") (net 2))
 (via (at 166.55 120.2) (size 0.6) (drill 0.3) (layers "F.Cu" "B.Cu") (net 2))
 (via (at 160.8 120.9) (size 0.6) (drill 0.3) (layers "F.Cu" "B.Cu") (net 2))
 (via (at 165.9 125.8) (size 0.4) (drill 0.2) (layers "F.Cu" "B.Cu") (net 2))
 (via (at 164.2 126.3) (size 0.4) (drill 0.2) (layers "F.Cu" "B.Cu") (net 2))
 (segment (start 156.999 120.648943) (end 159.551057 123.201) (width 0.2) (layer "B.Cu") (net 2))
 (segment (start 166.55 120.299943) (end 166.55 120.2) (width 0.2) (layer "B.Cu") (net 2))
 (segment (start 163.648943 123.201) (end 166.55 120.299943) (width 0.2) (layer "B.Cu") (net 2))
 (segment (start 159.551057 123.201) (end 163.648943 123.201) (width 0.2) (layer "B.Cu") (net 2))
 (segment (start 157.351057 119.799) (end 156.999 120.151057) (width 0.2) (layer "B.Cu") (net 2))
 (segment (start 159.699 119.799) (end 157.351057 119.799) (width 0.2) (layer "B.Cu") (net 2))
 (segment (start 160.8 120.9) (end 159.699 119.799) (width 0.2) (layer "B.Cu") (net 2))
 (segment (start 156.999 120.151057) (end 156.999 120.648943) (width 0.2) (layer "B.Cu") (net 2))
 (segment (start 165.4 126.3) (end 164.2 126.3) (width 0.1) (layer "B.Cu") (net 2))
 (segment (start 165.9 125.8) (end 165.4 126.3) (width 0.1) (layer "B.Cu") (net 2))
 (segment (start 155.899917 108.157791) (end 157.1 109.357874) (width 0.2) (layer "F.Cu") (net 3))
 (segment (start 157.1 119.349999) (end 156.049999 120.4) (width 0.2) (layer "F.Cu") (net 3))
 (segment (start 157.1 109.357874) (end 157.1 111.650001) (width 0.2) (layer "F.Cu") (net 3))
 (segment (start 157.1 111.650001) (end 157.1 117.949999) (width 0.2) (layer "F.Cu") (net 3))
 (segment (start 157.1 117.949999) (end 157.1 119.349999) (width 0.2) (layer "F.Cu") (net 3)))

